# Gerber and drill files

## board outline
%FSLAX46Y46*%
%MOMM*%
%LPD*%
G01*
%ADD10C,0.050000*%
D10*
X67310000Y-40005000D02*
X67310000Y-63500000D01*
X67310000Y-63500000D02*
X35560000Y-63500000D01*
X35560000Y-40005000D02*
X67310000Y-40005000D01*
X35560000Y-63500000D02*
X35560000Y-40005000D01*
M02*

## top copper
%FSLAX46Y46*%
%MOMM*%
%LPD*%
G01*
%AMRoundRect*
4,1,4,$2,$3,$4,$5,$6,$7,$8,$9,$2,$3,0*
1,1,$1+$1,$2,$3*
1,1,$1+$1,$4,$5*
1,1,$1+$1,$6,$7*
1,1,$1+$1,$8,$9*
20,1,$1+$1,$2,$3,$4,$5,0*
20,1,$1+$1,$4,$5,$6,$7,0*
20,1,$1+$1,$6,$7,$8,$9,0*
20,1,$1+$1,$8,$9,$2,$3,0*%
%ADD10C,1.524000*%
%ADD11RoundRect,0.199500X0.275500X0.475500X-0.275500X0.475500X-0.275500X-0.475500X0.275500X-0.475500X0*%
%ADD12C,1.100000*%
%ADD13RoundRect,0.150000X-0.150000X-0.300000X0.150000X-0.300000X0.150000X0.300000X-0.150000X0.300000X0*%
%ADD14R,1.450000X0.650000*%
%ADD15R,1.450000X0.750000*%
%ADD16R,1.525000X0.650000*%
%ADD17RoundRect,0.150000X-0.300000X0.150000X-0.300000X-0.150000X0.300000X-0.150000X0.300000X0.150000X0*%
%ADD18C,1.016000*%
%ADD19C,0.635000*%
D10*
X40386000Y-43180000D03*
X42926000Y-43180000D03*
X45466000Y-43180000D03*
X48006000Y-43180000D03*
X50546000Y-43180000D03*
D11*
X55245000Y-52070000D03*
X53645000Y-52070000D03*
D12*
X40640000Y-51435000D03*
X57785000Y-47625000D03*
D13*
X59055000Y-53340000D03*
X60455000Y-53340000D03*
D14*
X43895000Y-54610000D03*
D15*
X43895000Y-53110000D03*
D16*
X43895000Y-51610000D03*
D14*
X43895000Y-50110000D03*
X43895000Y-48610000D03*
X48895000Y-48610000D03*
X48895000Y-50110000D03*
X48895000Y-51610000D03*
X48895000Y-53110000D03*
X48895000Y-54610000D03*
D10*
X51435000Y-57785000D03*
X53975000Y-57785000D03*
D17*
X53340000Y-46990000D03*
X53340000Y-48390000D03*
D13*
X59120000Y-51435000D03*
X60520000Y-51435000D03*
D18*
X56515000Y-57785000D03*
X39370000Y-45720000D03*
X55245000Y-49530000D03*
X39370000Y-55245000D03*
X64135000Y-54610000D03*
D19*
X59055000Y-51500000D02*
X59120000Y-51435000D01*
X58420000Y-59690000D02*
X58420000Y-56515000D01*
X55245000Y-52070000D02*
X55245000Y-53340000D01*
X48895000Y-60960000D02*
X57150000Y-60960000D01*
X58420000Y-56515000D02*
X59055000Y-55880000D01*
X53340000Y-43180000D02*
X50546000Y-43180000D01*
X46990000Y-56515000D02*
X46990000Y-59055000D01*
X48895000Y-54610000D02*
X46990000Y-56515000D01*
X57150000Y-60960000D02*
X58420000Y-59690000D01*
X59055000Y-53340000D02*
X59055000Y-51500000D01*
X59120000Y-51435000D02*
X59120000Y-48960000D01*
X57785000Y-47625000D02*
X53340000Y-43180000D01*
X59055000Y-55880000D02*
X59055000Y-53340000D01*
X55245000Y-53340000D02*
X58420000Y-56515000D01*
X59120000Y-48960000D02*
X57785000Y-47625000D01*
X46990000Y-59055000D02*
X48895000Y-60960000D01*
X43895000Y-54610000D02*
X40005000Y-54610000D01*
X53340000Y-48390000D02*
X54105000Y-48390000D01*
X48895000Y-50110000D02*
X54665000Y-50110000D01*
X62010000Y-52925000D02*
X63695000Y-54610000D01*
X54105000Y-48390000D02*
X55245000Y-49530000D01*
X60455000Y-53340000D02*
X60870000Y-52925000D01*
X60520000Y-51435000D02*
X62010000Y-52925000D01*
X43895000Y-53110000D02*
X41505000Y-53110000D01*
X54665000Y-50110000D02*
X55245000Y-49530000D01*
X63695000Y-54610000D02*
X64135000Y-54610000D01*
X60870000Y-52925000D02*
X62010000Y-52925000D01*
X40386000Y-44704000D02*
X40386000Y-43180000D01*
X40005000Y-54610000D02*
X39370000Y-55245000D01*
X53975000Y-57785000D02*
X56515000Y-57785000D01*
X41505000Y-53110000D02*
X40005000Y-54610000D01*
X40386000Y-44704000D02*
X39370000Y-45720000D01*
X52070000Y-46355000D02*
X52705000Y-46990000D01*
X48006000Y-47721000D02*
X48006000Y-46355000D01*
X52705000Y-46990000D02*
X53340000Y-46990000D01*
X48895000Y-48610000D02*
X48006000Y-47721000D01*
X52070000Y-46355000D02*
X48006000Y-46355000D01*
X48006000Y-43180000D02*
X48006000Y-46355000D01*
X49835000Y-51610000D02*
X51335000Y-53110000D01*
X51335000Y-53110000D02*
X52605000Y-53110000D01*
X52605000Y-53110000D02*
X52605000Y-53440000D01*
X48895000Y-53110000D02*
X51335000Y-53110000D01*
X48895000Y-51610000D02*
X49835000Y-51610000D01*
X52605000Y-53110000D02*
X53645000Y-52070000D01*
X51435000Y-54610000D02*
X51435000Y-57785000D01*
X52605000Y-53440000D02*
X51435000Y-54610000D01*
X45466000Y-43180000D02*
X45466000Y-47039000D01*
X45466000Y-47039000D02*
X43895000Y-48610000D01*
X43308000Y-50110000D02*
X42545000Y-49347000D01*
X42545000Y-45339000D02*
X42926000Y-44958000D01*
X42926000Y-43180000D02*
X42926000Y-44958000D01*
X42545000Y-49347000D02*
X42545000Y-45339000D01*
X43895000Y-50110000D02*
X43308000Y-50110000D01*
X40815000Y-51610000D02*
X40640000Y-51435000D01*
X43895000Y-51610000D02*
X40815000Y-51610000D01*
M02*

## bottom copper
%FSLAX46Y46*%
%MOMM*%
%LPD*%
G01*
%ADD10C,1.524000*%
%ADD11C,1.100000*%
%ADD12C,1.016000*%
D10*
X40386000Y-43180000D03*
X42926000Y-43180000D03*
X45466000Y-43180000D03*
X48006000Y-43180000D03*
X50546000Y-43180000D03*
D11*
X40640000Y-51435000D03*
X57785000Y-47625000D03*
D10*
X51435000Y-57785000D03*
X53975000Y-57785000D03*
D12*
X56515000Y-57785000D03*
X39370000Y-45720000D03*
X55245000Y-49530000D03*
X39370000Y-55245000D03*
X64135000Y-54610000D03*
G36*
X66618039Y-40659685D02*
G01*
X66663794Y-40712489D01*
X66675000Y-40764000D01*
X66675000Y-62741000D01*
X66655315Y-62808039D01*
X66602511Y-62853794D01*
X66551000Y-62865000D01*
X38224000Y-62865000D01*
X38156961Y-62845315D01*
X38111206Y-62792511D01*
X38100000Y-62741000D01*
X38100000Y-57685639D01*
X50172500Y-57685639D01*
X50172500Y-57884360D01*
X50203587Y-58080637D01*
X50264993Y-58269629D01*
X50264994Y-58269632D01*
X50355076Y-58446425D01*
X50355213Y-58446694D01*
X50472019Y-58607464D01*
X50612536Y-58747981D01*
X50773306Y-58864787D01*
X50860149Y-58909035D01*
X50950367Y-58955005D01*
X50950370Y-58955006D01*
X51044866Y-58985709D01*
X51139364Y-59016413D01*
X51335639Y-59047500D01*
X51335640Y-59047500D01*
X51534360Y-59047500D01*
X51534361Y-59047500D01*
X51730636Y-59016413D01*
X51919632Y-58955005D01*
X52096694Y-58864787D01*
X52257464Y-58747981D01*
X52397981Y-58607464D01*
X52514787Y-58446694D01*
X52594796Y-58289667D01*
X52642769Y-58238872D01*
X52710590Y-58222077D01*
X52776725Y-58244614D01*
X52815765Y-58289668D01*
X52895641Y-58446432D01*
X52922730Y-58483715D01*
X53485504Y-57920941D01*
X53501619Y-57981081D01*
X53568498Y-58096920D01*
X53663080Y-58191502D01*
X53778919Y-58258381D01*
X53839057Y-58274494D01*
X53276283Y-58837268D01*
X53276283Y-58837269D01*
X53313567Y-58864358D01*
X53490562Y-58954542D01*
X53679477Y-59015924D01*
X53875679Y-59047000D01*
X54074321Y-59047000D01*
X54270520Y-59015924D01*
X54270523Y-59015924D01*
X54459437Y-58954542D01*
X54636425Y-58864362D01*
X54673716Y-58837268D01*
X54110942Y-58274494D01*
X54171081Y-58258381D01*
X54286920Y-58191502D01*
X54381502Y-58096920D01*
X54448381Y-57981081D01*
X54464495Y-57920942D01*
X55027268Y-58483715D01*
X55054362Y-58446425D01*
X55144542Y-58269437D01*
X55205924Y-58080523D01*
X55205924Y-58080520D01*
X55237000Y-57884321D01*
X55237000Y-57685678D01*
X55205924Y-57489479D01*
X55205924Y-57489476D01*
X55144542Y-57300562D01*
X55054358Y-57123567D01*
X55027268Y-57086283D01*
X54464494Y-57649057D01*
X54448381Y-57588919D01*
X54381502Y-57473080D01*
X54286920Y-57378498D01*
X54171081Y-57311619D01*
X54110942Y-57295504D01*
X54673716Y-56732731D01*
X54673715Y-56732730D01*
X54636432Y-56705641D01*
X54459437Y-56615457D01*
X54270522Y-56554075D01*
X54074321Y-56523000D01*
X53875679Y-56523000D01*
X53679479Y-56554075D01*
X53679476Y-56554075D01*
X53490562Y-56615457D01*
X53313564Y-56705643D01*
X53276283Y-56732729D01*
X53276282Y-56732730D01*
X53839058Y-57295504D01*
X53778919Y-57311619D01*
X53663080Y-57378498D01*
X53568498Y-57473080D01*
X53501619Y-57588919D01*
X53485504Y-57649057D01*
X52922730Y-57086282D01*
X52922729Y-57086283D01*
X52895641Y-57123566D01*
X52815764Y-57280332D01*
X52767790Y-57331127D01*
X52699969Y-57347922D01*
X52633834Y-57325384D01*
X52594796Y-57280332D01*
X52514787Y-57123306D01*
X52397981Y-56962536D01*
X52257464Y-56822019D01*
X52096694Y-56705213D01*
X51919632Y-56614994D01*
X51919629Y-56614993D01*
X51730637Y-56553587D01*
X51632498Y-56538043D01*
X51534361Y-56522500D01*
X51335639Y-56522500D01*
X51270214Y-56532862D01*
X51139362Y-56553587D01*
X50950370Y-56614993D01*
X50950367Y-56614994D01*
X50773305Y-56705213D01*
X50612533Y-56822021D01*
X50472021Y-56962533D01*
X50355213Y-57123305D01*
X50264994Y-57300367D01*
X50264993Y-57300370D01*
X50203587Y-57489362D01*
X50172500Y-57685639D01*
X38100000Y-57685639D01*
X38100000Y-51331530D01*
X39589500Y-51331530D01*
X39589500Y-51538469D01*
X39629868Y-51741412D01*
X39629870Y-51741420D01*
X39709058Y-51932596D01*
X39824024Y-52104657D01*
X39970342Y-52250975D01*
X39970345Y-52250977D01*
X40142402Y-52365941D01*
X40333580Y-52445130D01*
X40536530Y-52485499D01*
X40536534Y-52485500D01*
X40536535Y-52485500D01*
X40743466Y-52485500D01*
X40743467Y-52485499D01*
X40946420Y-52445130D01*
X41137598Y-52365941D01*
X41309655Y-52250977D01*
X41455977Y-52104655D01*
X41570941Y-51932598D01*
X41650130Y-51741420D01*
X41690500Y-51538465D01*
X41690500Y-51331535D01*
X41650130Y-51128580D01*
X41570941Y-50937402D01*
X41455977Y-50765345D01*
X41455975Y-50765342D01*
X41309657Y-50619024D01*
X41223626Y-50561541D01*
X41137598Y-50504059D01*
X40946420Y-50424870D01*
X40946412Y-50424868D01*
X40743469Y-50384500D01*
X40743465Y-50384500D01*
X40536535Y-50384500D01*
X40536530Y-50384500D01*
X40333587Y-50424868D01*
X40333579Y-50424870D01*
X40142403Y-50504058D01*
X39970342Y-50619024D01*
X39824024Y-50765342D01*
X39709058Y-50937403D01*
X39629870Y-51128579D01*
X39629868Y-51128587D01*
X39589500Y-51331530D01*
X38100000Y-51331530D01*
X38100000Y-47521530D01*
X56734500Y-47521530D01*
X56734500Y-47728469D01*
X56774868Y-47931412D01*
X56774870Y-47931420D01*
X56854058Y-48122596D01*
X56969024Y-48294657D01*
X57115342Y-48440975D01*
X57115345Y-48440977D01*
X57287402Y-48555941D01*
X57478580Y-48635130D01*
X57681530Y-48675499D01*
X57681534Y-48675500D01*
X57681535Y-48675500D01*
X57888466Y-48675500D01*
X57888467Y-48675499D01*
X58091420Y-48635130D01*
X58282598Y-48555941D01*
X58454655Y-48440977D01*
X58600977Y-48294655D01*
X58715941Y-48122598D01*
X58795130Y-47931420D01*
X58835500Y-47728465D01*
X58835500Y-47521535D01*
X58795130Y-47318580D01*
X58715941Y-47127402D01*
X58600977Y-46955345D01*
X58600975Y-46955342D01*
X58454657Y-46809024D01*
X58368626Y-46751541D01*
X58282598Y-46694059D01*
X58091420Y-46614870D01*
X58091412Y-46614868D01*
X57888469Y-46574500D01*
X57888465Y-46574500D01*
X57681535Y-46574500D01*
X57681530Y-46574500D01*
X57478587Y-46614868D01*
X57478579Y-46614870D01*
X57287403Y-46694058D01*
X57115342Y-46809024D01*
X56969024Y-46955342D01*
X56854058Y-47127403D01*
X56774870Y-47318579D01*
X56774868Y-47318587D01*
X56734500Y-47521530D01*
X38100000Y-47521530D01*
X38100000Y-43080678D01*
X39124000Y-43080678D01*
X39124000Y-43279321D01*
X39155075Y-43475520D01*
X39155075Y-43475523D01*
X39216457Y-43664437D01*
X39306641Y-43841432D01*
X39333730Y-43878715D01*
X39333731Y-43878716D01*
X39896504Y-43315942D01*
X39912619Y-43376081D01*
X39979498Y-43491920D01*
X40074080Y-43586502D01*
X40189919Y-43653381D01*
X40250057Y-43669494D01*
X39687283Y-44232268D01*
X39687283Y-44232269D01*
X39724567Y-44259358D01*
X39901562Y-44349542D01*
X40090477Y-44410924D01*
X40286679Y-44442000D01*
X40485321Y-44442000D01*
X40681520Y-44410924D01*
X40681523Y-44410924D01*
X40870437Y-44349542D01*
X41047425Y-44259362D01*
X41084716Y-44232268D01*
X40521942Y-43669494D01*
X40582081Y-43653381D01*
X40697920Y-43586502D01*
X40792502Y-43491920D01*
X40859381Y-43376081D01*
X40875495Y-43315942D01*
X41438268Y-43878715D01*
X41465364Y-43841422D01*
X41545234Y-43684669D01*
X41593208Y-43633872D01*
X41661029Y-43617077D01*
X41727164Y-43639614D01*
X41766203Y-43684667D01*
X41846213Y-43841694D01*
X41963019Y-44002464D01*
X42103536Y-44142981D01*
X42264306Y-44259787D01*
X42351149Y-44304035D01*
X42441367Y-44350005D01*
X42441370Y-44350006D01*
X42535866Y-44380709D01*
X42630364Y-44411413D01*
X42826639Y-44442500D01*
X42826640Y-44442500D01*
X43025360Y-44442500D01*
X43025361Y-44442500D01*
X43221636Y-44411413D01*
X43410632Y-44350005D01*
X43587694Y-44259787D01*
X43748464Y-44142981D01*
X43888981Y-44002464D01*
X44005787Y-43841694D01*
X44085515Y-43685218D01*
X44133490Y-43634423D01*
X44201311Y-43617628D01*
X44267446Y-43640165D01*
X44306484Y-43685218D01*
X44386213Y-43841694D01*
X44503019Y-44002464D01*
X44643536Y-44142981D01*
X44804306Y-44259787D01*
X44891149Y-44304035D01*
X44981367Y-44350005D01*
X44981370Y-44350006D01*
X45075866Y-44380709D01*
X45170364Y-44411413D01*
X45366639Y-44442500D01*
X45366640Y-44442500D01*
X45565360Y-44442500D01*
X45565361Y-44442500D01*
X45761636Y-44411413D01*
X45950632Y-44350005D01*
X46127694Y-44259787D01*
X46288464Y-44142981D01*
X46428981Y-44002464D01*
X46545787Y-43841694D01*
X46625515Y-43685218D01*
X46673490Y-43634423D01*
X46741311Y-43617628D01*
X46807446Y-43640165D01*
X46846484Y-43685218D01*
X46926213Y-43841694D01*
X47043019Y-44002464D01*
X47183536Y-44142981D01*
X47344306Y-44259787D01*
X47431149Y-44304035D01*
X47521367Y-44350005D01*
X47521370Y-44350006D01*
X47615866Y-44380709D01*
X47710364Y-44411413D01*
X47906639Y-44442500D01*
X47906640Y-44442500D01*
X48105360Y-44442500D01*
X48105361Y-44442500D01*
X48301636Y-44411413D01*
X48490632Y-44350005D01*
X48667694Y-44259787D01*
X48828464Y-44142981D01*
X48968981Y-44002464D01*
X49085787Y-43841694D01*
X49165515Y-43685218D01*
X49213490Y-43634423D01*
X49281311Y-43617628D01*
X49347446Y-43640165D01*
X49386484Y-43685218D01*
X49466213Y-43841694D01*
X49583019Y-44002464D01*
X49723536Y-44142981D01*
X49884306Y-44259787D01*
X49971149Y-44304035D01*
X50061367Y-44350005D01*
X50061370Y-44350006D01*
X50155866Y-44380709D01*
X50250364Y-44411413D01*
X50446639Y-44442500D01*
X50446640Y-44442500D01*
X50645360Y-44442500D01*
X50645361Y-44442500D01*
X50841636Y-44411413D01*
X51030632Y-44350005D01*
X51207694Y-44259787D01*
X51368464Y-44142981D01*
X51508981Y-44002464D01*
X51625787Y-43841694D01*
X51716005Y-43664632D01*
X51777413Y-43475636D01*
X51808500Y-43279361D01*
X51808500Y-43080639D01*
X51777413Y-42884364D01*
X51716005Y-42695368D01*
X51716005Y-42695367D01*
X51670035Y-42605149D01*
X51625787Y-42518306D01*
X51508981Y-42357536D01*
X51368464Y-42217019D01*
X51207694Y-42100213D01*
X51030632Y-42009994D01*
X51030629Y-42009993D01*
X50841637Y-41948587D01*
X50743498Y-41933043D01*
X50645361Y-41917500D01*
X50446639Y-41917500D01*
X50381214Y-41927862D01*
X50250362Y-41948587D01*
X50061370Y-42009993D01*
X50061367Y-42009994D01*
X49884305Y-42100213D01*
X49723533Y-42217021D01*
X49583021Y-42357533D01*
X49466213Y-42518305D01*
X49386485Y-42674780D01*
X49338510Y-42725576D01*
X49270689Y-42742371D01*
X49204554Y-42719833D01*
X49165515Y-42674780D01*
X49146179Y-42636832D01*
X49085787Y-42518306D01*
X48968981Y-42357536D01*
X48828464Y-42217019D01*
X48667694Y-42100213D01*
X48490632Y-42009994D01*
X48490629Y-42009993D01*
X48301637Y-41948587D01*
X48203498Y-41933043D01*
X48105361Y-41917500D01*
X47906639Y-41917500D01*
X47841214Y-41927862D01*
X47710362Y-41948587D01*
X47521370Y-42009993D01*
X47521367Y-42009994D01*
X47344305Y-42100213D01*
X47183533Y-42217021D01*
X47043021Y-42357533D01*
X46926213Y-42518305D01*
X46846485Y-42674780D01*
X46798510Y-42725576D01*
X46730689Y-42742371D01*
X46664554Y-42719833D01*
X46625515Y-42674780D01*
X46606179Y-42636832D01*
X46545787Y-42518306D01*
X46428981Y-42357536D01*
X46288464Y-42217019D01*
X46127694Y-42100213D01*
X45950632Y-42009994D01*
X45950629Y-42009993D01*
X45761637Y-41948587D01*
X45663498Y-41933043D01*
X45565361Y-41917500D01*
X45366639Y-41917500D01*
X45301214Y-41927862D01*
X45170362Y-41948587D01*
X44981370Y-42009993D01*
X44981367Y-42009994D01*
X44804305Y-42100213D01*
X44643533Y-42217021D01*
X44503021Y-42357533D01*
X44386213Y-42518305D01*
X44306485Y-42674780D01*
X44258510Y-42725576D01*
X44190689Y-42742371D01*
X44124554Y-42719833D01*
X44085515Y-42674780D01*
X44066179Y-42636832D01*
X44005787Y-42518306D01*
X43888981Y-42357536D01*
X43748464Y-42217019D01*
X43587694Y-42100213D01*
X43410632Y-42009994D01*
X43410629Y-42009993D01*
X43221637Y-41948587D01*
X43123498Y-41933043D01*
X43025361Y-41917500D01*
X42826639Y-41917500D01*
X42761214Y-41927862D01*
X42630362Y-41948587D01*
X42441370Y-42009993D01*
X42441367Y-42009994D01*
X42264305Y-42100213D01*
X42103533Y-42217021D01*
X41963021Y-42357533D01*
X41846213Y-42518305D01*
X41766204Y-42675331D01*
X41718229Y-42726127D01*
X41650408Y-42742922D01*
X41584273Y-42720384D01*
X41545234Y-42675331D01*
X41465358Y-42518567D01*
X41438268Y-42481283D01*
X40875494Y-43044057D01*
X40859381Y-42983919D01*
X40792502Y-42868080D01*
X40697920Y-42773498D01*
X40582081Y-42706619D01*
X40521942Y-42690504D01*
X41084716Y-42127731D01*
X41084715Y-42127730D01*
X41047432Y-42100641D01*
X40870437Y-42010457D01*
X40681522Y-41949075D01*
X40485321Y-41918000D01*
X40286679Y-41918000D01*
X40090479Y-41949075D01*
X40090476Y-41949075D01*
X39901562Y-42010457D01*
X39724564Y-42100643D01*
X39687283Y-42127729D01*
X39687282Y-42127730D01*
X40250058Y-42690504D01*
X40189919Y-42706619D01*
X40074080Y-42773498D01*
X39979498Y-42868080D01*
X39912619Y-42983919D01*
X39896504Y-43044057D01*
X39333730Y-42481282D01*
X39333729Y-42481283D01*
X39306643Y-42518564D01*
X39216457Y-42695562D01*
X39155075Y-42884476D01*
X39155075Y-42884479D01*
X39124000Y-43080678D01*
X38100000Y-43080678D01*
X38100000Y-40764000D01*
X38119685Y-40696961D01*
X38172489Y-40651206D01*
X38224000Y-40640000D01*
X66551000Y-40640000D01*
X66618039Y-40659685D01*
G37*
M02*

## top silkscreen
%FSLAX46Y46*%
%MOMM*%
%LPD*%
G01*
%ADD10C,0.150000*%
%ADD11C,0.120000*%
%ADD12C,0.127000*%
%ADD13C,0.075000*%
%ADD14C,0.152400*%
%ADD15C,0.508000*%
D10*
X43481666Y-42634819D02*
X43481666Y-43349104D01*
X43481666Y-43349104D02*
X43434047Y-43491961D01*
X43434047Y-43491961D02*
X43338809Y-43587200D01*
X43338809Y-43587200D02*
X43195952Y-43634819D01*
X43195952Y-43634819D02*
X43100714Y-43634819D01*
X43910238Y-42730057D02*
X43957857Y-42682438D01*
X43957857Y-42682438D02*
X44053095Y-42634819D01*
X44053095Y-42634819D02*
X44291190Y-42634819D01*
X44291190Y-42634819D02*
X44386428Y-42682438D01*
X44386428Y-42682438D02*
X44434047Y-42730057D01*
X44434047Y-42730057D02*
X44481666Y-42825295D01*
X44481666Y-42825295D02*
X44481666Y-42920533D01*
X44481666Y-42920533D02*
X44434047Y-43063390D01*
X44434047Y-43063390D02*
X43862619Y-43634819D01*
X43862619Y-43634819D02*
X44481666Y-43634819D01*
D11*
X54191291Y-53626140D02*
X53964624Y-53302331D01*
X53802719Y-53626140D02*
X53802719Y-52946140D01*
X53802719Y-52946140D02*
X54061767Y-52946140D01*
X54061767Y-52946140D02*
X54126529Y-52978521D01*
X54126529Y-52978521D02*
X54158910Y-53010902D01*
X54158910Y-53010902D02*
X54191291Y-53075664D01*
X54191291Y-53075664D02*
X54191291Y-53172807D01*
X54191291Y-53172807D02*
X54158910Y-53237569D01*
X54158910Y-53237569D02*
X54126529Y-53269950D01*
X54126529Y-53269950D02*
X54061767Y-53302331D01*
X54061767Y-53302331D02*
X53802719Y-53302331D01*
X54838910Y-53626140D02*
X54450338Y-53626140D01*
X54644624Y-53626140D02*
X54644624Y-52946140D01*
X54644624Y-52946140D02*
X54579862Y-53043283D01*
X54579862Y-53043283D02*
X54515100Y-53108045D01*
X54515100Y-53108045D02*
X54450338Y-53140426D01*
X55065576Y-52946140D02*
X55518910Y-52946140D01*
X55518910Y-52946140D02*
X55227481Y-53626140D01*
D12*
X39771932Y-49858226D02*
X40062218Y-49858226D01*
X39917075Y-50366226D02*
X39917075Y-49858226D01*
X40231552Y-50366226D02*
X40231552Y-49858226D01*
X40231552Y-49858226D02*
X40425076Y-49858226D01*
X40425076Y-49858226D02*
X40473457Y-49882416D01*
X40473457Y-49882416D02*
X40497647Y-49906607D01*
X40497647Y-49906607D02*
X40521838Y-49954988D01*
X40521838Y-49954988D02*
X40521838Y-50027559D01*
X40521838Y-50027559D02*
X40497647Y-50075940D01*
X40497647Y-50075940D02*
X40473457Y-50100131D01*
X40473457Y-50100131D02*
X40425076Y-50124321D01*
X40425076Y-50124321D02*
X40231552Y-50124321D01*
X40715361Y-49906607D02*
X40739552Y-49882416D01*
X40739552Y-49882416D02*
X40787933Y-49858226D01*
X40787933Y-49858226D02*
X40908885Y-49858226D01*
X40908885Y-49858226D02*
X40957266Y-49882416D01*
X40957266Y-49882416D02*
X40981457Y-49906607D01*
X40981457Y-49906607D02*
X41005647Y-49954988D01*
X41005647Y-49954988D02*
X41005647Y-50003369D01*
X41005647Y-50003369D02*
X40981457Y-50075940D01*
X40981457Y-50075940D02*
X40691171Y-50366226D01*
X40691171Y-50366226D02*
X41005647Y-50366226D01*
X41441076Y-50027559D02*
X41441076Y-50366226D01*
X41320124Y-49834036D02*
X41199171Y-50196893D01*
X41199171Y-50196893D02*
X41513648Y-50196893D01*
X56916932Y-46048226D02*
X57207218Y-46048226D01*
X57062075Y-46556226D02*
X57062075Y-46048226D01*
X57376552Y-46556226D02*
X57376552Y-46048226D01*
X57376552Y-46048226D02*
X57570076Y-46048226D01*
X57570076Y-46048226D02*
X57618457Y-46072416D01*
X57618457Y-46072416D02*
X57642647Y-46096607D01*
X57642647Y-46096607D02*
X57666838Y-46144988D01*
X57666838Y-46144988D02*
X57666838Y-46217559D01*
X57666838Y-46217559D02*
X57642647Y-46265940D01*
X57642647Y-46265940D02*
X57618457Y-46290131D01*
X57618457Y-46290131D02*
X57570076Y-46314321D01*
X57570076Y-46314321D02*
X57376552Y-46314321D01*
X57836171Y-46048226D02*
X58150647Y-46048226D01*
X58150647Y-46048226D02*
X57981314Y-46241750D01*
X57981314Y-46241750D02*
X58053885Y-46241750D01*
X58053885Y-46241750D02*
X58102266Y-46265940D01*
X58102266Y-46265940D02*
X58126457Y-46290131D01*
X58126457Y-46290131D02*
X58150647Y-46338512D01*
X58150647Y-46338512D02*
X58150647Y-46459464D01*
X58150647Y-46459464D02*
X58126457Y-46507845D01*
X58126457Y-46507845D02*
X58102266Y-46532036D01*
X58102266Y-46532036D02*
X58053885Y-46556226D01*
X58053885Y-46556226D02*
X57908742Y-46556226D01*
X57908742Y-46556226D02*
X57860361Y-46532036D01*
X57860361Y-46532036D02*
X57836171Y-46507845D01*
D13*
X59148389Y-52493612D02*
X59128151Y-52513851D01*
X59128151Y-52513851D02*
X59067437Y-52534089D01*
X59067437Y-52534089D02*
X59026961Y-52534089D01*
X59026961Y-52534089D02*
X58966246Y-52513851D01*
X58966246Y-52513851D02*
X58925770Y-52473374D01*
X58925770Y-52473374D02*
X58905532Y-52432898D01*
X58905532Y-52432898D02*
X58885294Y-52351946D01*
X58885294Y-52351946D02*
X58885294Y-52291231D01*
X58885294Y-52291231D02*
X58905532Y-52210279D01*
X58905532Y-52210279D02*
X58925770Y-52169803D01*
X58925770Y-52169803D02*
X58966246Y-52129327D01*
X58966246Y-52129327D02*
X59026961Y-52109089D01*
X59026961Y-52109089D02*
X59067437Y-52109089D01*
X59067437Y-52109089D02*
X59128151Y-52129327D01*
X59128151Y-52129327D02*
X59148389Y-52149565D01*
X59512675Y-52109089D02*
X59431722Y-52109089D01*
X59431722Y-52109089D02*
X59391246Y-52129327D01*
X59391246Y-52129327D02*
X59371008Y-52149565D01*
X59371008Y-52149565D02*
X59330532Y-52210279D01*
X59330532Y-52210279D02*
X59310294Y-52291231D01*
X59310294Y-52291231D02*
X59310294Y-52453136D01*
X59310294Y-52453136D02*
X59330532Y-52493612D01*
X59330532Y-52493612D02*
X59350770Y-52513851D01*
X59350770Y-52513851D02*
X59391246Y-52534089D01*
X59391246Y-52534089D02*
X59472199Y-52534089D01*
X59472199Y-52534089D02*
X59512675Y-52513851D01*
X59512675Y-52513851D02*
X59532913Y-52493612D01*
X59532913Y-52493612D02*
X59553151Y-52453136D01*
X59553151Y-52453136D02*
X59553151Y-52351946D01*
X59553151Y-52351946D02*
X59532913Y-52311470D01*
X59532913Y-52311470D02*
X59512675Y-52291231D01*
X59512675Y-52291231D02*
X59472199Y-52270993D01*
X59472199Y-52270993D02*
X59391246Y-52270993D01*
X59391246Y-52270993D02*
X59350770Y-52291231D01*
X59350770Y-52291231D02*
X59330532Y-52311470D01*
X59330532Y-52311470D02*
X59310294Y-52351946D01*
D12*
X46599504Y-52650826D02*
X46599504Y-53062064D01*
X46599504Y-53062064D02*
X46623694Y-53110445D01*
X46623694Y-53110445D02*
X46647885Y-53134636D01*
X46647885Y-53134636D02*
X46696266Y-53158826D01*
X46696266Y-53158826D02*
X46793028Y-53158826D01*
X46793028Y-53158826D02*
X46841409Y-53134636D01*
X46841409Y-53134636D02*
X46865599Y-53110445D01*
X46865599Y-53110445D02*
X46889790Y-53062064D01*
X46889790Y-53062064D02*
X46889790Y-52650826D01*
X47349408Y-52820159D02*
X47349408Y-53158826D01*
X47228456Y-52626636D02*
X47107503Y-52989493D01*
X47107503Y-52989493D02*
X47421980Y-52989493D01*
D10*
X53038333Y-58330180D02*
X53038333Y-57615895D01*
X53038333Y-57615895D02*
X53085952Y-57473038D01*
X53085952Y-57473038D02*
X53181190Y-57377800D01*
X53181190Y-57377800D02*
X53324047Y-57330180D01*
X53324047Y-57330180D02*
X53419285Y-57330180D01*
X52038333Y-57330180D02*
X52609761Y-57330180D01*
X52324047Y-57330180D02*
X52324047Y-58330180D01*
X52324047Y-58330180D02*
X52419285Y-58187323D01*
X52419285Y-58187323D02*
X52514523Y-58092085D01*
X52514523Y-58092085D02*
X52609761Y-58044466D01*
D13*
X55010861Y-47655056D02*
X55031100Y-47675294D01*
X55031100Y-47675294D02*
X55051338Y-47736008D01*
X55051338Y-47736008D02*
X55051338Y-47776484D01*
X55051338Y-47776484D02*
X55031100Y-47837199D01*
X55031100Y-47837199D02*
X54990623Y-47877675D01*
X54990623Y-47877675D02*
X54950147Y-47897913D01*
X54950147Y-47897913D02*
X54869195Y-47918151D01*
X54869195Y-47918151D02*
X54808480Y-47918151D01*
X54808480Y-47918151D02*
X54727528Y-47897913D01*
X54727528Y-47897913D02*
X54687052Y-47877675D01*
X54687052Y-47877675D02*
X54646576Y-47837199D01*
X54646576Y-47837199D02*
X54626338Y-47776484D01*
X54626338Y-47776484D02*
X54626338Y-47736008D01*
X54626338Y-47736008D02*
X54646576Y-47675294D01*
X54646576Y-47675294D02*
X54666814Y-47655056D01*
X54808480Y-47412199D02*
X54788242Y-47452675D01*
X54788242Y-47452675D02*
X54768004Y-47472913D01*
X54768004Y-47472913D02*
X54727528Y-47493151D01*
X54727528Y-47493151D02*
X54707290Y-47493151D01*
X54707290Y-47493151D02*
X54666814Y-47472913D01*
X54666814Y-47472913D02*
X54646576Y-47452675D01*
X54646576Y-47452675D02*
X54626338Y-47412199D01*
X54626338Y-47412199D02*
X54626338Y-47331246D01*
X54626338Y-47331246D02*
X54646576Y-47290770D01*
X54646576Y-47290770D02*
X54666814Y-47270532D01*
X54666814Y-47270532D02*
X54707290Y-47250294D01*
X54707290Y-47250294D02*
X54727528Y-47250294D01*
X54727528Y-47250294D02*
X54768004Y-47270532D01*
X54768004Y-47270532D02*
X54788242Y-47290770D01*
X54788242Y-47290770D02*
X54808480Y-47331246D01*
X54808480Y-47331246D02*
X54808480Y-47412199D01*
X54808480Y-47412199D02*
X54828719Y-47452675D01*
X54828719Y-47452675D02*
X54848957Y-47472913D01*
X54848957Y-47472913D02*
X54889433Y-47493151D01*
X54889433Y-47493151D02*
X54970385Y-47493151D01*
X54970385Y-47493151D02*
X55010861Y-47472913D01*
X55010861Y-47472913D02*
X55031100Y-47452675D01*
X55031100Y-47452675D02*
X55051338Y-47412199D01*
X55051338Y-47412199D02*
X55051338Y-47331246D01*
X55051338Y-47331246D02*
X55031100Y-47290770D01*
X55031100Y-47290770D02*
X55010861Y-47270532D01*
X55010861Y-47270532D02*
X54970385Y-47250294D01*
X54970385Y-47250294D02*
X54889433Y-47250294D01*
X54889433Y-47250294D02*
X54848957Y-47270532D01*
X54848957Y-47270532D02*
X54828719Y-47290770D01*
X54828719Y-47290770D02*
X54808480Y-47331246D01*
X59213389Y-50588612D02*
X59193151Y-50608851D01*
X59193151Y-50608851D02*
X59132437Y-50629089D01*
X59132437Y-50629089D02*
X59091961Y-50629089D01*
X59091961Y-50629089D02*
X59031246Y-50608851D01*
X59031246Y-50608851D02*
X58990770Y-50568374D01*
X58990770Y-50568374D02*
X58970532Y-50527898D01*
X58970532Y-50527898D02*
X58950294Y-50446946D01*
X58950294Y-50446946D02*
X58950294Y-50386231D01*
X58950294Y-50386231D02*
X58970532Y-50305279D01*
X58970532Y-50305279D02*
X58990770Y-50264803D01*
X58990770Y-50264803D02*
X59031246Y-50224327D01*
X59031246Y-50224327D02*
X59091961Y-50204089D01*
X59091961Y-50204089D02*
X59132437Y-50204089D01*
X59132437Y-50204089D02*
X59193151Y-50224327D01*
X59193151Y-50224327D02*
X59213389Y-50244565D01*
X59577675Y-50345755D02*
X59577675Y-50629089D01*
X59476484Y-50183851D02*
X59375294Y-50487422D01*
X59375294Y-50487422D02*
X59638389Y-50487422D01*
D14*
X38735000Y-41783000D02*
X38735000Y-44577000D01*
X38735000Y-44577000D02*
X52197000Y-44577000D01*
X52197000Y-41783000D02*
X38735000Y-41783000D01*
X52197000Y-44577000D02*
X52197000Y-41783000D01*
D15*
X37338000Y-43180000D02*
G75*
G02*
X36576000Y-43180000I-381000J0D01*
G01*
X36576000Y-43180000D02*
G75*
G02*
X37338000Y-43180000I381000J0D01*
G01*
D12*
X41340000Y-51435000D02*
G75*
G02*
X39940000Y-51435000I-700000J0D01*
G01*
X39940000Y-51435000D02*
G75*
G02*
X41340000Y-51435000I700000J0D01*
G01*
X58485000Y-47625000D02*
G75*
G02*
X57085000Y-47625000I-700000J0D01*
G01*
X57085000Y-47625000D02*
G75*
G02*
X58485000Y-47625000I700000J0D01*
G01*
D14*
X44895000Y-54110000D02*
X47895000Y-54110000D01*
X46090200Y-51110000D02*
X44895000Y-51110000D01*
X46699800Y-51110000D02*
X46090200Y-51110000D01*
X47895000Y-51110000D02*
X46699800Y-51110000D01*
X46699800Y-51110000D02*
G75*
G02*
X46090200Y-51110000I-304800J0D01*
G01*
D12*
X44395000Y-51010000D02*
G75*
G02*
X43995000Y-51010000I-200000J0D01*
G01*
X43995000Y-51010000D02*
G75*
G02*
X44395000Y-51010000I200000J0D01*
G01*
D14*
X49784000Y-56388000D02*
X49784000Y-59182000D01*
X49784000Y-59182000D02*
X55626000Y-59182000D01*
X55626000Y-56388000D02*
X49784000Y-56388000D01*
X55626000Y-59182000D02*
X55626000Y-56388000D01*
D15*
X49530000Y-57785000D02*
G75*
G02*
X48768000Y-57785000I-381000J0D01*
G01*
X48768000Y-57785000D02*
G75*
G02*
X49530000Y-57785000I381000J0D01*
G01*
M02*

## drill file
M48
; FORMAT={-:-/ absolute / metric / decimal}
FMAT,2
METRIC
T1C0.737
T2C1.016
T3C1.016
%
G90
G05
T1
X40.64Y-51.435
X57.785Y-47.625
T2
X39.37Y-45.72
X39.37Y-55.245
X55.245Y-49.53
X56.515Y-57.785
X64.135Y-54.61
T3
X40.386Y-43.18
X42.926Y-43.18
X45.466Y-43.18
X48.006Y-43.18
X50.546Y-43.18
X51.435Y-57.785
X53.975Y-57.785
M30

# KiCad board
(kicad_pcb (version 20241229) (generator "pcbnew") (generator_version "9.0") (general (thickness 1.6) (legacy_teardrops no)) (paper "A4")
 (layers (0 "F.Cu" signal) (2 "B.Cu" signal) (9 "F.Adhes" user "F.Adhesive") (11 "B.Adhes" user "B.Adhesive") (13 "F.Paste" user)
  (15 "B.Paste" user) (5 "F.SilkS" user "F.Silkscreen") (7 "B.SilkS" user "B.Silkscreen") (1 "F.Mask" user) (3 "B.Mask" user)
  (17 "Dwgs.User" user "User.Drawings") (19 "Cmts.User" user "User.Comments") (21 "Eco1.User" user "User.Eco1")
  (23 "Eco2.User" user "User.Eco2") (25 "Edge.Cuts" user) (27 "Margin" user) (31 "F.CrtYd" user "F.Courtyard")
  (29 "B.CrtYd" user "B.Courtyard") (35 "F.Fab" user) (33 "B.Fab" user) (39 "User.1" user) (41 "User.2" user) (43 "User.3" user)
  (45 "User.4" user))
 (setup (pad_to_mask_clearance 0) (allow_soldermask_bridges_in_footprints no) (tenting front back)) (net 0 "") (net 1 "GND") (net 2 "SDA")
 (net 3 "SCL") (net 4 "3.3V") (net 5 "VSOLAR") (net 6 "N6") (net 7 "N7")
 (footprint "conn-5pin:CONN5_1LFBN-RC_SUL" (layer "F.Cu") (at 40.386 43.18)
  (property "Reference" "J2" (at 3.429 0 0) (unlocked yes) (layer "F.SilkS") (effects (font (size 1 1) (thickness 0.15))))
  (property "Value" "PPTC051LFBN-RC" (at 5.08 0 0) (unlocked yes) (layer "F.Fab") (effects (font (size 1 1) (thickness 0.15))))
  (fp_line (start -1.651 -1.397) (end -1.651 1.397) (stroke (width 0.1524) (type solid)) (layer "F.SilkS"))
  (fp_line (start -1.651 1.397) (end 11.811 1.397) (stroke (width 0.1524) (type solid)) (layer "F.SilkS"))
  (fp_line (start 11.811 -1.397) (end -1.651 -1.397) (stroke (width 0.1524) (type solid)) (layer "F.SilkS"))
  (fp_line (start 11.811 1.397) (end 11.811 -1.397) (stroke (width 0.1524) (type solid)) (layer "F.SilkS"))
  (fp_circle (center -3.429 0) (end -3.048 0) (stroke (width 0.508) (type solid)) (fill no) (layer "F.SilkS"))
  (pad "1" thru_hole circle (at 0 0) (size 1.524 1.524) (drill 1.016) (layers "*.Cu" "*.Mask") (remove_unused_layers no) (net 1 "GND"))
  (pad "2" thru_hole circle (at 2.54 0) (size 1.524 1.524) (drill 1.016) (layers "*.Cu" "*.Mask") (remove_unused_layers no) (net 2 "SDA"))
  (pad "3" thru_hole circle (at 5.08 0) (size 1.524 1.524) (drill 1.016) (layers "*.Cu" "*.Mask") (remove_unused_layers no) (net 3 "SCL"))
  (pad "4" thru_hole circle (at 7.62 0) (size 1.524 1.524) (drill 1.016) (layers "*.Cu" "*.Mask") (remove_unused_layers no) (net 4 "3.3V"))
  (pad "5" thru_hole circle (at 10.16 0) (size 1.524 1.524) (drill 1.016) (layers "*.Cu" "*.Mask") (remove_unused_layers no)
   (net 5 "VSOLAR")))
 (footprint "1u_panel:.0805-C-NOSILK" (layer "F.Cu") (at 54.445 52.07 180)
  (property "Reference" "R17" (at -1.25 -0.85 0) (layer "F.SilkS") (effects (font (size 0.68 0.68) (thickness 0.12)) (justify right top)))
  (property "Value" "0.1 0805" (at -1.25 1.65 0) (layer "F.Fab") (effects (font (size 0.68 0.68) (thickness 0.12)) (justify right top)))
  (pad "1" smd roundrect (at -0.8 0 180) (size 0.95 1.35) (layers "F.Cu" "F.Paste") (roundrect_rratio 0.21) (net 5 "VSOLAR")
   (solder_mask_margin 0.0635) (thermal_bridge_angle 45))
  (pad "2" smd roundrect (at 0.8 0 180) (size 0.95 1.35) (layers "F.Cu" "F.Paste") (roundrect_rratio 0.21) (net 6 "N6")
   (solder_mask_margin 0.0635) (thermal_bridge_angle 45)))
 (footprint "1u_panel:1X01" (layer "F.Cu") (at 40.64 51.435)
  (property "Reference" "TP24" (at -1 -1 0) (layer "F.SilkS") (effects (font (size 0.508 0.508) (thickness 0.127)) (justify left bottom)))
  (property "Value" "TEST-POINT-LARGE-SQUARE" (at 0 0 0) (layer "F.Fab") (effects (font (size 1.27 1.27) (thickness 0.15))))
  (fp_circle (center 0 0) (end 0.7 0) (stroke (width 0.127) (type solid)) (fill no) (layer "F.SilkS"))
  (pad "1" thru_hole circle (at 0 0) (size 1.1 1.1) (drill 0.7366) (layers "*.Cu" "*.Mask") (remove_unused_layers no) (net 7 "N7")
   (solder_mask_margin 0.0635)))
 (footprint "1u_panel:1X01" (layer "F.Cu") (at 57.785 47.625)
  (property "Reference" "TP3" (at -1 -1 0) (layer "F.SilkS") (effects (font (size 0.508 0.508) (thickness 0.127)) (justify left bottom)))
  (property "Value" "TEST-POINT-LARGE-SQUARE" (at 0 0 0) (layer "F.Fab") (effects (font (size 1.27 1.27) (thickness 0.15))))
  (fp_circle (center 0 0) (end 0.7 0) (stroke (width 0.127) (type solid)) (fill no) (layer "F.SilkS"))
  (pad "1" thru_hole circle (at 0 0) (size 1.1 1.1) (drill 0.7366) (layers "*.Cu" "*.Mask") (remove_unused_layers no) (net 5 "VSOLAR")
   (solder_mask_margin 0.0635)))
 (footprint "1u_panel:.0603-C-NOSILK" (layer "F.Cu") (at 59.755 53.34)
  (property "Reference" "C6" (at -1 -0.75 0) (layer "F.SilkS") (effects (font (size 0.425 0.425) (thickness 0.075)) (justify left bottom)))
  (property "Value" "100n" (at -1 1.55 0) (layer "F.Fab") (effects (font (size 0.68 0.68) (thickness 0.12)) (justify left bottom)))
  (pad "1" smd roundrect (at -0.7 0) (size 0.6 0.9) (layers "F.Cu" "F.Paste") (roundrect_rratio 0.25) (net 5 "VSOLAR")
   (solder_mask_margin 0.0635) (thermal_bridge_angle 45))
  (pad "2" smd roundrect (at 0.7 0) (size 0.6 0.9) (layers "F.Cu" "F.Paste") (roundrect_rratio 0.25) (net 1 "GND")
   (solder_mask_margin 0.0635) (thermal_bridge_angle 45)))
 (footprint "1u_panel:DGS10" (layer "F.Cu") (at 46.395 52.61)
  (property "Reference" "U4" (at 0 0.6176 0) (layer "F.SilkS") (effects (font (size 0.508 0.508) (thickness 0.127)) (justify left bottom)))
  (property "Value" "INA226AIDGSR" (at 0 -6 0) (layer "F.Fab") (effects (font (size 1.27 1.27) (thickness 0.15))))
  (fp_line (start -1.5 1.5) (end 1.5 1.5) (stroke (width 0.1524) (type solid)) (layer "F.SilkS"))
  (fp_line (start -0.3048 -1.5) (end -1.5 -1.5) (stroke (width 0.1524) (type solid)) (layer "F.SilkS"))
  (fp_line (start 0.3048 -1.5) (end -0.3048 -1.5) (stroke (width 0.1524) (type solid)) (layer "F.SilkS"))
  (fp_line (start 1.5 -1.5) (end 0.3048 -1.5) (stroke (width 0.1524) (type solid)) (layer "F.SilkS"))
  (fp_arc (start 0.3048 -1.5) (mid 0 -1.1952) (end -0.3048 -1.5) (stroke (width 0.1524) (type solid)) (layer "F.SilkS"))
  (fp_circle (center -2.2 -1.6) (end -2 -1.6) (stroke (width 0.127) (type solid)) (fill no) (layer "F.SilkS"))
  (pad "1" smd rect (at -2.5 2) (size 1.45 0.65) (layers "F.Cu" "F.Mask" "F.Paste") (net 1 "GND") (solder_mask_margin 0.0635)
   (thermal_bridge_angle 45))
  (pad "2" smd rect (at -2.5 0.5) (size 1.45 0.75) (layers "F.Cu" "F.Mask" "F.Paste") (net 1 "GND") (solder_mask_margin 0.0635)
   (thermal_bridge_angle 45))
  (pad "3" smd rect (at -2.5 -1) (size 1.525 0.65) (layers "F.Cu" "F.Mask" "F.Paste") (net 7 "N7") (solder_mask_margin 0.0635)
   (thermal_bridge_angle 45))
  (pad "4" smd rect (at -2.5 -2.5) (size 1.45 0.65) (layers "F.Cu" "F.Mask" "F.Paste") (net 2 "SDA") (solder_mask_margin 0.0635)
   (thermal_bridge_angle 45))
  (pad "5" smd rect (at -2.5 -4) (size 1.45 0.65) (layers "F.Cu" "F.Mask" "F.Paste") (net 3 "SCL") (solder_mask_margin 0.0635)
   (thermal_bridge_angle 45))
  (pad "6" smd rect (at 2.5 -4) (size 1.45 0.65) (layers "F.Cu" "F.Mask" "F.Paste") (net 4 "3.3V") (solder_mask_margin 0.0635)
   (thermal_bridge_angle 45))
  (pad "7" smd rect (at 2.5 -2.5) (size 1.45 0.65) (layers "F.Cu" "F.Mask" "F.Paste") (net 1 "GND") (solder_mask_margin 0.0635)
   (thermal_bridge_angle 45))
  (pad "8" smd rect (at 2.5 -1) (size 1.45 0.65) (layers "F.Cu" "F.Mask" "F.Paste") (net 6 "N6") (solder_mask_margin 0.0635)
   (thermal_bridge_angle 45))
  (pad "9" smd rect (at 2.5 0.5) (size 1.45 0.65) (layers "F.Cu" "F.Mask" "F.Paste") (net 6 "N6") (solder_mask_margin 0.0635)
   (thermal_bridge_angle 45))
  (pad "10" smd rect (at 2.5 2) (size 1.45 0.65) (layers "F.Cu" "F.Mask" "F.Paste") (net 5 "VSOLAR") (solder_mask_margin 0.0635)
   (thermal_bridge_angle 45)))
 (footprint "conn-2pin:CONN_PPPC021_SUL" (layer "F.Cu") (at 51.435 57.785 180)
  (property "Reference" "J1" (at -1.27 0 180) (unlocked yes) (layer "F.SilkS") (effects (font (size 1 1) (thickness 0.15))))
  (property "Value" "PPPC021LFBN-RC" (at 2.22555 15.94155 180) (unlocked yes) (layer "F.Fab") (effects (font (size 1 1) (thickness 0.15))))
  (fp_line (start 1.651 1.397) (end 1.651 -1.397) (stroke (width 0.1524) (type solid)) (layer "F.SilkS"))
  (fp_line (start 1.651 -1.397) (end -4.191 -1.397) (stroke (width 0.1524) (type solid)) (layer "F.SilkS"))
  (fp_line (start -4.191 1.397) (end 1.651 1.397) (stroke (width 0.1524) (type solid)) (layer "F.SilkS"))
  (fp_line (start -4.191 -1.397) (end -4.191 1.397) (stroke (width 0.1524) (type solid)) (layer "F.SilkS"))
  (fp_circle (center 2.286 0) (end 2.667 0) (stroke (width 0.508) (type solid)) (fill no) (layer "F.SilkS"))
  (pad "1" thru_hole circle (at 0 0 180) (size 1.524 1.524) (drill 1.016) (layers "*.Cu" "*.Mask") (remove_unused_layers no) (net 6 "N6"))
  (pad "2" thru_hole circle (at -2.54 0 180) (size 1.524 1.524) (drill 1.016) (layers "*.Cu" "*.Mask") (remove_unused_layers no)
   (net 1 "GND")))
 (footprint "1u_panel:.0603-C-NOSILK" (layer "F.Cu") (at 53.34 47.69 -90)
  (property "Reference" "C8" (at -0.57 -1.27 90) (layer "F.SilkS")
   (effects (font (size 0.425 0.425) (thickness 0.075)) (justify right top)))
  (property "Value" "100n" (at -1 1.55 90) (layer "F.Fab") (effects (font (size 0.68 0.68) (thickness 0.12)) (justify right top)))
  (pad "1" smd roundrect (at -0.7 0 270) (size 0.6 0.9) (layers "F.Cu" "F.Paste") (roundrect_rratio 0.25) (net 4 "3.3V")
   (solder_mask_margin 0.0635) (thermal_bridge_angle 45))
  (pad "2" smd roundrect (at 0.7 0 270) (size 0.6 0.9) (layers "F.Cu" "F.Paste") (roundrect_rratio 0.25) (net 1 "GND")
   (solder_mask_margin 0.0635) (thermal_bridge_angle 45)))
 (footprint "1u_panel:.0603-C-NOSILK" (layer "F.Cu") (at 59.82 51.435)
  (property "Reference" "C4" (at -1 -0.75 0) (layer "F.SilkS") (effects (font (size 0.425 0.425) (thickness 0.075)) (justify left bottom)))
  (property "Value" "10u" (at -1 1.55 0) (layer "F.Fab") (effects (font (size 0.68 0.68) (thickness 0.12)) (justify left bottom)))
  (pad "1" smd roundrect (at -0.7 0) (size 0.6 0.9) (layers "F.Cu" "F.Paste") (roundrect_rratio 0.25) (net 5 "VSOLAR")
   (solder_mask_margin 0.0635) (thermal_bridge_angle 45))
  (pad "2" smd roundrect (at 0.7 0) (size 0.6 0.9) (layers "F.Cu" "F.Paste") (roundrect_rratio 0.25) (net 1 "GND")
   (solder_mask_margin 0.0635) (thermal_bridge_angle 45)))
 (gr_line (start 67.31 40.005) (end 67.31 63.5) (stroke (width 0.05) (type default)) (layer "Edge.Cuts"))
 (gr_line (start 67.31 63.5) (end 35.56 63.5) (stroke (width 0.05) (type default)) (layer "Edge.Cuts"))
 (gr_line (start 35.56 40.005) (end 67.31 40.005) (stroke (width 0.05) (type default)) (layer "Edge.Cuts"))
 (gr_line (start 35.56 63.5) (end 35.56 40.005) (stroke (width 0.05) (type default)) (layer "Edge.Cuts"))
 (segment (start 59.055 51.5) (end 59.12 51.435) (width 0.635) (layer "F.Cu") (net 5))
 (segment (start 58.42 59.69) (end 58.42 56.515) (width 0.635) (layer "F.Cu") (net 5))
 (segment (start 55.245 52.07) (end 55.245 53.34) (width 0.635) (layer "F.Cu") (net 5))
 (segment (start 48.895 60.96) (end 57.15 60.96) (width 0.635) (layer "F.Cu") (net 5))
 (segment (start 58.42 56.515) (end 59.055 55.88) (width 0.635) (layer "F.Cu") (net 5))
 (segment (start 53.34 43.18) (end 50.546 43.18) (width 0.635) (layer "F.Cu") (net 5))
 (segment (start 46.99 56.515) (end 46.99 59.055) (width 0.635) (layer "F.Cu") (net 5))
 (segment (start 48.895 54.61) (end 46.99 56.515) (width 0.635) (layer "F.Cu") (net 5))
 (segment (start 57.15 60.96) (end 58.42 59.69) (width 0.635) (layer "F.Cu") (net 5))
 (segment (start 59.055 53.34) (end 59.055 51.5) (width 0.635) (layer "F.Cu") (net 5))
 (segment (start 59.12 51.435) (end 59.12 48.96) (width 0.635) (layer "F.Cu") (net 5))
 (segment (start 57.785 47.625) (end 53.34 43.18) (width 0.635) (layer "F.Cu") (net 5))
 (segment (start 59.055 55.88) (end 59.055 53.34) (width 0.635) (layer "F.Cu") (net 5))
 (segment (start 55.245 53.34) (end 58.42 56.515) (width 0.635) (layer "F.Cu") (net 5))
 (segment (start 59.12 48.96) (end 57.785 47.625) (width 0.635) (layer "F.Cu") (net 5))
 (segment (start 46.99 59.055) (end 48.895 60.96) (width 0.635) (layer "F.Cu") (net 5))
 (segment (start 43.895 54.61) (end 40.005 54.61) (width 0.635) (layer "F.Cu") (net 1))
 (segment (start 53.34 48.39) (end 54.105 48.39) (width 0.635) (layer "F.Cu") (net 1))
 (segment (start 48.895 50.11) (end 54.665 50.11) (width 0.635) (layer "F.Cu") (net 1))
 (segment (start 62.01 52.925) (end 63.695 54.61) (width 0.635) (layer "F.Cu") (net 1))
 (segment (start 54.105 48.39) (end 55.245 49.53) (width 0.635) (layer "F.Cu") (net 1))
 (segment (start 60.455 53.34) (end 60.87 52.925) (width 0.635) (layer "F.Cu") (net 1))
 (segment (start 60.52 51.435) (end 62.01 52.925) (width 0.635) (layer "F.Cu") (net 1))
 (segment (start 43.895 53.11) (end 41.505 53.11) (width 0.635) (layer "F.Cu") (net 1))
 (segment (start 54.665 50.11) (end 55.245 49.53) (width 0.635) (layer "F.Cu") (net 1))
 (segment (start 63.695 54.61) (end 64.135 54.61) (width 0.635) (layer "F.Cu") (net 1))
 (segment (start 60.87 52.925) (end 62.01 52.925) (width 0.635) (layer "F.Cu") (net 1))
 (segment (start 40.386 44.704) (end 40.386 43.18) (width 0.635) (layer "F.Cu") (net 1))
 (segment (start 40.005 54.61) (end 39.37 55.245) (width 0.635) (layer "F.Cu") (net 1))
 (segment (start 53.975 57.785) (end 56.515 57.785) (width 0.635) (layer "F.Cu") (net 1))
 (segment (start 41.505 53.11) (end 40.005 54.61) (width 0.635) (layer "F.Cu") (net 1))
 (segment (start 40.386 44.704) (end 39.37 45.72) (width 0.635) (layer "F.Cu") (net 1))
 (via (at 56.515 57.785) (size 1.016) (drill 1.016) (layers "F.Cu" "B.Cu") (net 1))
 (via (at 39.37 45.72) (size 1.016) (drill 1.016) (layers "F.Cu" "B.Cu") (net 1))
 (via (at 55.245 49.53) (size 1.016) (drill 1.016) (layers "F.Cu" "B.Cu") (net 1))
 (via (at 39.37 55.245) (size 1.016) (drill 1.016) (layers "F.Cu" "B.Cu") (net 1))
 (via (at 64.135 54.61) (size 1.016) (drill 1.016) (layers "F.Cu" "B.Cu") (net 1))
 (segment (start 52.07 46.355) (end 52.705 46.99) (width 0.635) (layer "F.Cu") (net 4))
 (segment (start 48.006 47.721) (end 48.006 46.355) (width 0.635) (layer "F.Cu") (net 4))
 (segment (start 52.705 46.99) (end 53.34 46.99) (width 0.635) (layer "F.Cu") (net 4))
 (segment (start 48.895 48.61) (end 48.006 47.721) (width 0.635) (layer "F.Cu") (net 4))
 (segment (start 52.07 46.355) (end 48.006 46.355) (width 0.635) (layer "F.Cu") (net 4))
 (segment (start 48.006 43.18) (end 48.006 46.355) (width 0.635) (layer "F.Cu") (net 4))
 (segment (start 49.835 51.61) (end 51.335 53.11) (width 0.635) (layer "F.Cu") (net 6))
 (segment (start 51.335 53.11) (end 52.605 53.11) (width 0.635) (layer "F.Cu") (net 6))
 (segment (start 52.605 53.11) (end 52.605 53.44) (width 0.635) (layer "F.Cu") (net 6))
 (segment (start 48.895 53.11) (end 51.335 53.11) (width 0.635) (layer "F.Cu") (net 6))
 (segment (start 48.895 51.61) (end 49.835 51.61) (width 0.635) (layer "F.Cu") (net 6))
 (segment (start 52.605 53.11) (end 53.645 52.07) (width 0.635) (layer "F.Cu") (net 6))
 (segment (start 51.435 54.61) (end 51.435 57.785) (width 0.635) (layer "F.Cu") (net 6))
 (segment (start 52.605 53.44) (end 51.435 54.61) (width 0.635) (layer "F.Cu") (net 6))
 (segment (start 45.466 43.18) (end 45.466 47.039) (width 0.635) (layer "F.Cu") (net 3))
 (segment (start 45.466 47.039) (end 43.895 48.61) (width 0.635) (layer "F.Cu") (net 3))
 (segment (start 43.308 50.11) (end 42.545 49.347) (width 0.635) (layer "F.Cu") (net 2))
 (segment (start 42.545 45.339) (end 42.926 44.958) (width 0.635) (layer "F.Cu") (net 2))
 (segment (start 42.926 43.18) (end 42.926 44.958) (width 0.635) (layer "F.Cu") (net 2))
 (segment (start 42.545 49.347) (end 42.545 45.339) (width 0.635) (layer "F.Cu") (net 2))
 (segment (start 43.895 50.11) (end 43.308 50.11) (width 0.635) (layer "F.Cu") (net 2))
 (segment (start 40.815 51.61) (end 40.64 51.435) (width 0.635) (layer "F.Cu") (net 7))
 (segment (start 43.895 51.61) (end 40.815 51.61) (width 0.635) (layer "F.Cu") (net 7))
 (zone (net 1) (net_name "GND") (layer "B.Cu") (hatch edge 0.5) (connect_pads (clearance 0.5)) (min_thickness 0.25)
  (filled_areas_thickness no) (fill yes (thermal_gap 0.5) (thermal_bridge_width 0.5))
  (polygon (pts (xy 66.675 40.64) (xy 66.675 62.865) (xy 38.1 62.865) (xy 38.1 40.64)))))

